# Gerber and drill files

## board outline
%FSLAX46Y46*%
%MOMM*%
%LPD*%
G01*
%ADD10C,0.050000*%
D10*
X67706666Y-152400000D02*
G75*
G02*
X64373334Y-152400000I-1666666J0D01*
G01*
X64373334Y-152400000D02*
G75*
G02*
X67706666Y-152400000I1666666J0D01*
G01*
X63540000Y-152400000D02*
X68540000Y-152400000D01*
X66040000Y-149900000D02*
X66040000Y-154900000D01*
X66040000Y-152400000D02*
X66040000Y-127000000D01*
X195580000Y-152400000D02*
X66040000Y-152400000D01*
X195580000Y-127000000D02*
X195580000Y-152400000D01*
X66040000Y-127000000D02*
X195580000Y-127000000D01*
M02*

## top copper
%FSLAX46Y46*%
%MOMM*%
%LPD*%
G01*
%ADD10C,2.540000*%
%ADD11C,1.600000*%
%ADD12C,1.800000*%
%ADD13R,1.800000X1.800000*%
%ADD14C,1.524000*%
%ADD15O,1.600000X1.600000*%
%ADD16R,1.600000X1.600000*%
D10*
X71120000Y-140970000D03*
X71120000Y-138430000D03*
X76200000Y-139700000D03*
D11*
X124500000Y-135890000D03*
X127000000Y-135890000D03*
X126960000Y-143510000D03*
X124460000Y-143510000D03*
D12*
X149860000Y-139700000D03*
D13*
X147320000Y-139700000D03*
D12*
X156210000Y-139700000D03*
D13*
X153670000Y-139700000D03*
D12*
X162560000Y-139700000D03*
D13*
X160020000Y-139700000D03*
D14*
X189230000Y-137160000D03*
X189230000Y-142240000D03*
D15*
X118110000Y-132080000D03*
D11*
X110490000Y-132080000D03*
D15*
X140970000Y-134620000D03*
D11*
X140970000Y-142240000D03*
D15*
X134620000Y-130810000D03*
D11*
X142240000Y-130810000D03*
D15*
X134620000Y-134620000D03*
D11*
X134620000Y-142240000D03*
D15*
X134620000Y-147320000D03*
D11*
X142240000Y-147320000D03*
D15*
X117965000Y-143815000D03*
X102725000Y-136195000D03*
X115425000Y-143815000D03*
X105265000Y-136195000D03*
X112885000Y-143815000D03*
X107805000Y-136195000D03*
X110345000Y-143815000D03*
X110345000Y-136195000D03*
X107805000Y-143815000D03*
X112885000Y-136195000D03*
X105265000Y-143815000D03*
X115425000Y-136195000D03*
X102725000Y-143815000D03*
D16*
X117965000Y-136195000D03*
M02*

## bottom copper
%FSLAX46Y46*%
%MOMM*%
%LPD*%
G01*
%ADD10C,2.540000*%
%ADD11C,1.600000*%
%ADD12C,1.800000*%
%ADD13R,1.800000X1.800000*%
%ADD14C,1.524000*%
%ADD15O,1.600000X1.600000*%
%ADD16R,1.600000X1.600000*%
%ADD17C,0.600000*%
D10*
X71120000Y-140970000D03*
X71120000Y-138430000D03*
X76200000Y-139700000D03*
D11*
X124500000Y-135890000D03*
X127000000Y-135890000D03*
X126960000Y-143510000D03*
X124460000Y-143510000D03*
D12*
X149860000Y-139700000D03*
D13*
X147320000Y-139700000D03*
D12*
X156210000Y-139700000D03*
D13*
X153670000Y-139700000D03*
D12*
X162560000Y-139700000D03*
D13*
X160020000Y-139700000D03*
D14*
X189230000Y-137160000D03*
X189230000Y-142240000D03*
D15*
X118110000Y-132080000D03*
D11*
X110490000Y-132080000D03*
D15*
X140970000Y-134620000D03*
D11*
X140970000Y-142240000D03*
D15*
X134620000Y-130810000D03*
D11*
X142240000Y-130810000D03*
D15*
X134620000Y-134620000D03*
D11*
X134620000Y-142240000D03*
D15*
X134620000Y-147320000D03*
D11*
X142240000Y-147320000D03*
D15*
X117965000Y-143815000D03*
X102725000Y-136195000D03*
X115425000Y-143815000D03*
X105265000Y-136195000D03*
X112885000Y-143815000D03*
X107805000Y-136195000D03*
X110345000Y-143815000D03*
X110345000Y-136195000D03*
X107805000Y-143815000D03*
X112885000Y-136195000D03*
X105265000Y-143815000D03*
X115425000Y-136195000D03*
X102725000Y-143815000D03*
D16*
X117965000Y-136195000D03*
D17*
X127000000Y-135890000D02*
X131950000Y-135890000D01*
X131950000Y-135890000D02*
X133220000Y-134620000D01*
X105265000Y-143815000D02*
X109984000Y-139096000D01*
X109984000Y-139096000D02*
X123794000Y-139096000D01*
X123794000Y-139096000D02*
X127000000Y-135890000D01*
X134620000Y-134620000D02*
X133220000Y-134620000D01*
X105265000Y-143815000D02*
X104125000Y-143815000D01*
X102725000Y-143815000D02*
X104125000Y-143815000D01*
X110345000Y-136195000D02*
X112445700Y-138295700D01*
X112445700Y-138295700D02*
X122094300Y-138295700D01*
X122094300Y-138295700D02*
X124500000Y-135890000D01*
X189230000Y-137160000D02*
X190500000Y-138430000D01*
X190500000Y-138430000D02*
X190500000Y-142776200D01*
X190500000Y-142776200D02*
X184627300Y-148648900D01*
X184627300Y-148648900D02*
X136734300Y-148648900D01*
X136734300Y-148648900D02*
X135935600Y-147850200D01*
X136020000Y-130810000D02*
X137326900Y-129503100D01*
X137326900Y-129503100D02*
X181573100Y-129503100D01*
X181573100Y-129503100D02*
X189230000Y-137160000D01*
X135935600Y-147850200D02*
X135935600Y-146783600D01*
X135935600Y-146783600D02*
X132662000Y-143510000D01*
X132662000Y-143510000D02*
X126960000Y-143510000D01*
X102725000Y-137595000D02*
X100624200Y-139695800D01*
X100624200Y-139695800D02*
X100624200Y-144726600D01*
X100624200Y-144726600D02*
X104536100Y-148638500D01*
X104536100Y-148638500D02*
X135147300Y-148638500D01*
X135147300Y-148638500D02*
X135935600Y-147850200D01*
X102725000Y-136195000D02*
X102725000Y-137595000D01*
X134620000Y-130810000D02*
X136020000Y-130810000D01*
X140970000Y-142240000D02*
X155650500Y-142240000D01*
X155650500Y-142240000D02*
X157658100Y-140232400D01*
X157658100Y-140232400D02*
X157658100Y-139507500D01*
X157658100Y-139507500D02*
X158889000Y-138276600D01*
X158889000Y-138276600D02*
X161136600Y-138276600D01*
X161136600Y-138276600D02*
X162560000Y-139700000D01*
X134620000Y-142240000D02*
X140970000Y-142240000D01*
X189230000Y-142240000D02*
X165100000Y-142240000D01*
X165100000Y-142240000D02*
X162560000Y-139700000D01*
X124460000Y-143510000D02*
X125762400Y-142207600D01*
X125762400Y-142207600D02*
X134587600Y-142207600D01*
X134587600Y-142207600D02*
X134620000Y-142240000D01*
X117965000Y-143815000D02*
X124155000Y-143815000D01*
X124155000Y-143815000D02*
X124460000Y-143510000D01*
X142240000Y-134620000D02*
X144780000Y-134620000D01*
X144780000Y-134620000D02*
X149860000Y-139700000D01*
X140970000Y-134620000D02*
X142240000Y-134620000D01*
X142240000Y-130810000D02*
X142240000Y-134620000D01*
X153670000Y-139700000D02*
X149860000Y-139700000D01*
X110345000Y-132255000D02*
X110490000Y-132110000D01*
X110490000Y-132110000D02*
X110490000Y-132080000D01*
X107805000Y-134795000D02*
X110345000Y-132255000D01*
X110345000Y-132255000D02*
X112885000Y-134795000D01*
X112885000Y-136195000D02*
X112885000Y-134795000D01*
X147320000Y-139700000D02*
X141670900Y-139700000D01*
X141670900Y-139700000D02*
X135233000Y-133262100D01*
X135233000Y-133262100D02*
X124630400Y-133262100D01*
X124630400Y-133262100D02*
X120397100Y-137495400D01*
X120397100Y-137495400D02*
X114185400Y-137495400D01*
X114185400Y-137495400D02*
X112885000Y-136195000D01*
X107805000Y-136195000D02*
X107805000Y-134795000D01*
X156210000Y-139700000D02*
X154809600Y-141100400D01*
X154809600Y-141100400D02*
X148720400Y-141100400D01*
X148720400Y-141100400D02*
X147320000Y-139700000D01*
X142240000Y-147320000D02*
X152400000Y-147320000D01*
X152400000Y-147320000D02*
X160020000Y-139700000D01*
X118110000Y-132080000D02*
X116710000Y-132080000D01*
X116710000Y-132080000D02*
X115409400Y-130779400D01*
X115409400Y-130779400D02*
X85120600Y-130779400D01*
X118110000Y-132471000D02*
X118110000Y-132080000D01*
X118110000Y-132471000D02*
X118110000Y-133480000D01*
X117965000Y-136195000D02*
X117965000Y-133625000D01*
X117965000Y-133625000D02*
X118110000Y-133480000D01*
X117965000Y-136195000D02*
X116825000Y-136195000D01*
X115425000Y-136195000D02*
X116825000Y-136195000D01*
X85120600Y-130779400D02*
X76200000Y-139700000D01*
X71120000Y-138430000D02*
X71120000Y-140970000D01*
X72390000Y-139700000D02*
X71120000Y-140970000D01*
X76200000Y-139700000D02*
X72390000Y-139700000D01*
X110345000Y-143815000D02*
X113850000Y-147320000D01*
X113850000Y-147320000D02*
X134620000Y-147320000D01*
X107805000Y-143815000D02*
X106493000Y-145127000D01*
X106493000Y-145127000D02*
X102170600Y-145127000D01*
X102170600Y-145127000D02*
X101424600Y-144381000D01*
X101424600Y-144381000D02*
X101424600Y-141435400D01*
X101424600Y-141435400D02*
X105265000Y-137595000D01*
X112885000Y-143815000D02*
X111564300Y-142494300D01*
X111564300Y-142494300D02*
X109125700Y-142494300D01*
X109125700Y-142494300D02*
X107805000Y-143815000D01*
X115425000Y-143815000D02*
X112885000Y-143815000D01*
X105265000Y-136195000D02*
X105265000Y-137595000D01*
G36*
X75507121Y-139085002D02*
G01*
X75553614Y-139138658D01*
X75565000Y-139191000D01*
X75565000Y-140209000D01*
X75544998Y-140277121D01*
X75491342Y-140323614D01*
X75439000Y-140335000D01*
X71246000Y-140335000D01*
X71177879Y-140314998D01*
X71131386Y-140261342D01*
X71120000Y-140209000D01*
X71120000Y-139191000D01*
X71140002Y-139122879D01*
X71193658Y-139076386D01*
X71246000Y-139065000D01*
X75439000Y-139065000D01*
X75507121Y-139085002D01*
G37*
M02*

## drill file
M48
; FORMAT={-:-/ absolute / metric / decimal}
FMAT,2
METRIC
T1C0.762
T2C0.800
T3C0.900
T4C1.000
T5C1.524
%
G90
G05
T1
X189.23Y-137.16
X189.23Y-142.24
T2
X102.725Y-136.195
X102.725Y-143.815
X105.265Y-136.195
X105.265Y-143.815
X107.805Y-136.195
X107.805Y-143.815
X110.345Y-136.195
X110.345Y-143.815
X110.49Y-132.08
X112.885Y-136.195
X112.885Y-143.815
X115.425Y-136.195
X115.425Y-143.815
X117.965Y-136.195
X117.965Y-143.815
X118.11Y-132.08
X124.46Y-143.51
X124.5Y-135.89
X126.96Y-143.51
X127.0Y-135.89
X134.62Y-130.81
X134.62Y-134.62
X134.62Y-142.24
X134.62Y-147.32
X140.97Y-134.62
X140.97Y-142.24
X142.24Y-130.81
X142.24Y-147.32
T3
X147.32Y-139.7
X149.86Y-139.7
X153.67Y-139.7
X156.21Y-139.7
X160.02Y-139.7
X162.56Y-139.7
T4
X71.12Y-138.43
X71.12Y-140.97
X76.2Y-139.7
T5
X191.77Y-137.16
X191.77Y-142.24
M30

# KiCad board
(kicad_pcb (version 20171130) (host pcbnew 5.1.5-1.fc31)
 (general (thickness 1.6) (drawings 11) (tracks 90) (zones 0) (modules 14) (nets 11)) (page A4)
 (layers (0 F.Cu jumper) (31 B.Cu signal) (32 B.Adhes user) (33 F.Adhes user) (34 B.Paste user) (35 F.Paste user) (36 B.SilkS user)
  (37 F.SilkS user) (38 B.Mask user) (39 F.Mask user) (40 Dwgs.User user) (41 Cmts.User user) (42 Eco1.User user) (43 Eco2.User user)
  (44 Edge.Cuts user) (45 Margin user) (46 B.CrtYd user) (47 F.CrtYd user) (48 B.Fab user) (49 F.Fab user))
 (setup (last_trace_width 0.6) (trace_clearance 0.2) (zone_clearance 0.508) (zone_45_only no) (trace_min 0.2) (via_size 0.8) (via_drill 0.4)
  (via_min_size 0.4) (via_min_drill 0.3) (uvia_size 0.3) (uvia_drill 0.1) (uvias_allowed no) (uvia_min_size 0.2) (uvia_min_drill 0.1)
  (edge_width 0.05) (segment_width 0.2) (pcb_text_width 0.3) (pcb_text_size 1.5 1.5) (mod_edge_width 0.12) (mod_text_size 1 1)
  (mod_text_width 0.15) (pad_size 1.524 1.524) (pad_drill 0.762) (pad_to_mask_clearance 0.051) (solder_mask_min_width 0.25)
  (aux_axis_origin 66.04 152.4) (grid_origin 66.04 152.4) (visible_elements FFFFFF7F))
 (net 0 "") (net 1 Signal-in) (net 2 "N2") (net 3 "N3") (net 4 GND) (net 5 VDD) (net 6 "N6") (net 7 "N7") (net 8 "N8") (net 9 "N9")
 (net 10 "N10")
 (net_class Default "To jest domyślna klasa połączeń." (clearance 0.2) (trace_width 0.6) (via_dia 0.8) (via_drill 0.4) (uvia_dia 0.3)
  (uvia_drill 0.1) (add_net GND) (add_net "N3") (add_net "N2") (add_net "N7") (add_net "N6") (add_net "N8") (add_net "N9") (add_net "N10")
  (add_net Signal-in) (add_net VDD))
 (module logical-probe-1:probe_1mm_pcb (layer F.Cu) (at 76.2 139.7)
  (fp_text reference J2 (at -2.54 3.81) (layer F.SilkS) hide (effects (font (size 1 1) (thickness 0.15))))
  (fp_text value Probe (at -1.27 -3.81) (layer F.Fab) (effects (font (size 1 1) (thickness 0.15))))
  (pad 1 thru_hole circle (at -5.08 1.27) (size 2.54 2.54) (drill 1) (layers B.Cu B.Mask) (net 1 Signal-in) (zone_connect 2))
  (pad 1 thru_hole circle (at -5.08 -1.27) (size 2.54 2.54) (drill 1) (layers B.Cu B.Mask) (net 1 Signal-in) (zone_connect 2))
  (pad 1 thru_hole circle (at 0 0) (size 2.54 2.54) (drill 1) (layers B.Cu B.Mask) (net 1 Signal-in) (zone_connect 2)))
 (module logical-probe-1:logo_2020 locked (layer F.Cu) (at 175.26 147.32)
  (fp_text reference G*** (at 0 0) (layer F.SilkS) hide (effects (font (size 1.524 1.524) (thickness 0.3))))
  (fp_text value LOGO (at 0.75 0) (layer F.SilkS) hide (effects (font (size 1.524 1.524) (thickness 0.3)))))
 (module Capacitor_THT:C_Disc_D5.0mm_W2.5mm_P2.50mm (layer F.Cu) (at 127 135.89 180)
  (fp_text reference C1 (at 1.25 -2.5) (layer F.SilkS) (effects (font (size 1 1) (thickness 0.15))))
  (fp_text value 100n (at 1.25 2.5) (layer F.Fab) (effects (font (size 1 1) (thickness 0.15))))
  (pad 2 thru_hole circle (at 2.5 0 180) (size 1.6 1.6) (drill 0.8) (layers *.Cu *.Mask) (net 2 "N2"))
  (pad 1 thru_hole circle (at 0 0 180) (size 1.6 1.6) (drill 0.8) (layers *.Cu *.Mask) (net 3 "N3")))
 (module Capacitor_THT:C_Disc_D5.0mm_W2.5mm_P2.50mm (layer F.Cu) (at 124.46 143.51)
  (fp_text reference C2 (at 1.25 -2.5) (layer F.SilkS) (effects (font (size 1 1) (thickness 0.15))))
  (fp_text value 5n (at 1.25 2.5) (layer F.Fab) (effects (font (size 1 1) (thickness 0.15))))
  (pad 2 thru_hole circle (at 2.5 0) (size 1.6 1.6) (drill 0.8) (layers *.Cu *.Mask) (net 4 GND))
  (pad 1 thru_hole circle (at 0 0) (size 1.6 1.6) (drill 0.8) (layers *.Cu *.Mask) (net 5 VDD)))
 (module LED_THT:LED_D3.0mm (layer F.Cu) (at 147.32 139.7)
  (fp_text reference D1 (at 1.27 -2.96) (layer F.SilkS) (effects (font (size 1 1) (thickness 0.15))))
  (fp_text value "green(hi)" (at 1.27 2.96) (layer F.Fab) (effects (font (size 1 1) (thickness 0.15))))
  (pad 2 thru_hole circle (at 2.54 0) (size 1.8 1.8) (drill 0.9) (layers *.Cu *.Mask) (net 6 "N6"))
  (pad 1 thru_hole rect (at 0 0) (size 1.8 1.8) (drill 0.9) (layers *.Cu *.Mask) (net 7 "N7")))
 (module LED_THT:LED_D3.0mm (layer F.Cu) (at 153.67 139.7)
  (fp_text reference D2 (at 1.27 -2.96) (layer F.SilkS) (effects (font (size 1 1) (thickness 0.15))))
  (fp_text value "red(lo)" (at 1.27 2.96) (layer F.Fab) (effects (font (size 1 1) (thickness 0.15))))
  (pad 2 thru_hole circle (at 2.54 0) (size 1.8 1.8) (drill 0.9) (layers *.Cu *.Mask) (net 7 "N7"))
  (pad 1 thru_hole rect (at 0 0) (size 1.8 1.8) (drill 0.9) (layers *.Cu *.Mask) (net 6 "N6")))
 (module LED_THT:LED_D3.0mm (layer F.Cu) (at 160.02 139.7)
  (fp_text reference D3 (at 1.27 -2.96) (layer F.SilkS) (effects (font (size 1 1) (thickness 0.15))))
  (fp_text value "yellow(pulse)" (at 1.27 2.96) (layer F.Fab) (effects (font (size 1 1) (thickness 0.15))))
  (pad 2 thru_hole circle (at 2.54 0) (size 1.8 1.8) (drill 0.9) (layers *.Cu *.Mask) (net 5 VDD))
  (pad 1 thru_hole rect (at 0 0) (size 1.8 1.8) (drill 0.9) (layers *.Cu *.Mask) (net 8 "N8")))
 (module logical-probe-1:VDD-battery (layer F.Cu) (at 189.23 139.7)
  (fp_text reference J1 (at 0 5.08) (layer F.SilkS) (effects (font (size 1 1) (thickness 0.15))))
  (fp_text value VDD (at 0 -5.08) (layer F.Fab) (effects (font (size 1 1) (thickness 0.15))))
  (pad "" np_thru_hole circle (at 2.54 2.54) (size 1.524 1.524) (drill 1.524) (layers *.Cu *.Mask))
  (pad "" np_thru_hole circle (at 2.54 -2.54) (size 1.524 1.524) (drill 1.524) (layers *.Cu *.Mask))
  (pad 2 thru_hole circle (at 0 -2.54) (size 1.524 1.524) (drill 0.762) (layers *.Cu *.Mask) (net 4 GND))
  (pad 1 thru_hole circle (at 0 2.54) (size 1.524 1.524) (drill 0.762) (layers *.Cu *.Mask) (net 5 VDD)))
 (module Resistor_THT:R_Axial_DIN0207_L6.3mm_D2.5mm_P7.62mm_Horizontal (layer F.Cu) (at 110.49 132.08)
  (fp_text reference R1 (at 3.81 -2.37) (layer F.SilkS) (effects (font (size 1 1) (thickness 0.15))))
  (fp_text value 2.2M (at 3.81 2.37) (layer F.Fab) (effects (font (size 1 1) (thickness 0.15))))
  (pad 2 thru_hole oval (at 7.62 0) (size 1.6 1.6) (drill 0.8) (layers *.Cu *.Mask) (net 1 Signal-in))
  (pad 1 thru_hole circle (at 0 0) (size 1.6 1.6) (drill 0.8) (layers *.Cu *.Mask) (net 7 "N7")))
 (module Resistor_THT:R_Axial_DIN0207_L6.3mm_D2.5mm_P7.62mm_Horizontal (layer F.Cu) (at 140.97 142.24 90)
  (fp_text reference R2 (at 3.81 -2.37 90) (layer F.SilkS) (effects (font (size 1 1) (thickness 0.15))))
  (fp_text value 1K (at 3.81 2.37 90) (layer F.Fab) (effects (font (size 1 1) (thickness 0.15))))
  (pad 2 thru_hole oval (at 7.62 0 90) (size 1.6 1.6) (drill 0.8) (layers *.Cu *.Mask) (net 6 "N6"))
  (pad 1 thru_hole circle (at 0 0 90) (size 1.6 1.6) (drill 0.8) (layers *.Cu *.Mask) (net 5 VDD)))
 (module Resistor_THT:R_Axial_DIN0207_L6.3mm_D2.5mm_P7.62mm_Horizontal (layer F.Cu) (at 142.24 130.81 180)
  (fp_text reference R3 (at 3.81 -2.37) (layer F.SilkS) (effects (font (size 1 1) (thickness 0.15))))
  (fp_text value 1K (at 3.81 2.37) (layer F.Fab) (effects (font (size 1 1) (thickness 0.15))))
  (pad 2 thru_hole oval (at 7.62 0 180) (size 1.6 1.6) (drill 0.8) (layers *.Cu *.Mask) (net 4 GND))
  (pad 1 thru_hole circle (at 0 0 180) (size 1.6 1.6) (drill 0.8) (layers *.Cu *.Mask) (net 6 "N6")))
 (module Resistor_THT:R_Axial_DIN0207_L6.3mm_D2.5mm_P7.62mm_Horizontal (layer F.Cu) (at 134.62 142.24 90)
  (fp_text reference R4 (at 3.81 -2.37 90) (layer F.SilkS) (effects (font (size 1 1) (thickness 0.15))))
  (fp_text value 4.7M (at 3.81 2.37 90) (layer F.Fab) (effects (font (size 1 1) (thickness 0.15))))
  (pad 2 thru_hole oval (at 7.62 0 90) (size 1.6 1.6) (drill 0.8) (layers *.Cu *.Mask) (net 3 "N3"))
  (pad 1 thru_hole circle (at 0 0 90) (size 1.6 1.6) (drill 0.8) (layers *.Cu *.Mask) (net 5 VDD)))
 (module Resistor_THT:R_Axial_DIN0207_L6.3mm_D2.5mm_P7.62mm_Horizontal (layer F.Cu) (at 142.24 147.32 180)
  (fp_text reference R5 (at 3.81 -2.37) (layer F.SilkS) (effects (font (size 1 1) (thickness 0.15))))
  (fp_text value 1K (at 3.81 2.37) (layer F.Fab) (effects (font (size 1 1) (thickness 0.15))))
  (pad 2 thru_hole oval (at 7.62 0 180) (size 1.6 1.6) (drill 0.8) (layers *.Cu *.Mask) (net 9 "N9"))
  (pad 1 thru_hole circle (at 0 0 180) (size 1.6 1.6) (drill 0.8) (layers *.Cu *.Mask) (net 8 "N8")))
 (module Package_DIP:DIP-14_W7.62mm (layer F.Cu) (at 117.965 136.195 270)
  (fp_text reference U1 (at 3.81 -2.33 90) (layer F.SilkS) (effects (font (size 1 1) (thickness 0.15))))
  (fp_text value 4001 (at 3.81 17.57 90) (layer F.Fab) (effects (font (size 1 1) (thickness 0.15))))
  (pad 14 thru_hole oval (at 7.62 0 270) (size 1.6 1.6) (drill 0.8) (layers *.Cu *.Mask) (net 5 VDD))
  (pad 7 thru_hole oval (at 0 15.24 270) (size 1.6 1.6) (drill 0.8) (layers *.Cu *.Mask) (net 4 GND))
  (pad 13 thru_hole oval (at 7.62 2.54 270) (size 1.6 1.6) (drill 0.8) (layers *.Cu *.Mask) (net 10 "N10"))
  (pad 6 thru_hole oval (at 0 12.7 270) (size 1.6 1.6) (drill 0.8) (layers *.Cu *.Mask) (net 10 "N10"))
  (pad 12 thru_hole oval (at 7.62 5.08 270) (size 1.6 1.6) (drill 0.8) (layers *.Cu *.Mask) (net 10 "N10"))
  (pad 5 thru_hole oval (at 0 10.16 270) (size 1.6 1.6) (drill 0.8) (layers *.Cu *.Mask) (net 7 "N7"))
  (pad 11 thru_hole oval (at 7.62 7.62 270) (size 1.6 1.6) (drill 0.8) (layers *.Cu *.Mask) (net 9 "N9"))
  (pad 4 thru_hole oval (at 0 7.62 270) (size 1.6 1.6) (drill 0.8) (layers *.Cu *.Mask) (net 2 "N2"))
  (pad 10 thru_hole oval (at 7.62 10.16 270) (size 1.6 1.6) (drill 0.8) (layers *.Cu *.Mask) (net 10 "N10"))
  (pad 3 thru_hole oval (at 0 5.08 270) (size 1.6 1.6) (drill 0.8) (layers *.Cu *.Mask) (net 7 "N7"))
  (pad 9 thru_hole oval (at 7.62 12.7 270) (size 1.6 1.6) (drill 0.8) (layers *.Cu *.Mask) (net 3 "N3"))
  (pad 2 thru_hole oval (at 0 2.54 270) (size 1.6 1.6) (drill 0.8) (layers *.Cu *.Mask) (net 1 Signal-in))
  (pad 8 thru_hole oval (at 7.62 15.24 270) (size 1.6 1.6) (drill 0.8) (layers *.Cu *.Mask) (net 3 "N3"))
  (pad 1 thru_hole rect (at 0 0 270) (size 1.6 1.6) (drill 0.8) (layers *.Cu *.Mask) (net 1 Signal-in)))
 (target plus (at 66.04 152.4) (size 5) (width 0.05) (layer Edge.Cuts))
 (gr_line (start 66.04 152.4) (end 66.04 127) (layer Edge.Cuts) (width 0.05))
 (gr_line (start 195.58 152.4) (end 66.04 152.4) (layer Edge.Cuts) (width 0.05))
 (gr_line (start 195.58 127) (end 195.58 152.4) (layer Edge.Cuts) (width 0.05))
 (gr_line (start 66.04 127) (end 195.58 127) (layer Edge.Cuts) (width 0.05))
 (segment (start 127 135.89) (end 131.95 135.89) (width 0.6) (layer B.Cu) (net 3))
 (segment (start 131.95 135.89) (end 133.22 134.62) (width 0.6) (layer B.Cu) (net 3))
 (segment (start 105.265 143.815) (end 109.984 139.096) (width 0.6) (layer B.Cu) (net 3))
 (segment (start 109.984 139.096) (end 123.794 139.096) (width 0.6) (layer B.Cu) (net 3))
 (segment (start 123.794 139.096) (end 127 135.89) (width 0.6) (layer B.Cu) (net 3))
 (segment (start 134.62 134.62) (end 133.22 134.62) (width 0.6) (layer B.Cu) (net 3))
 (segment (start 105.265 143.815) (end 104.125 143.815) (width 0.6) (layer B.Cu) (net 3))
 (segment (start 102.725 143.815) (end 104.125 143.815) (width 0.6) (layer B.Cu) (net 3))
 (segment (start 110.345 136.195) (end 112.4457 138.2957) (width 0.6) (layer B.Cu) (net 2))
 (segment (start 112.4457 138.2957) (end 122.0943 138.2957) (width 0.6) (layer B.Cu) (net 2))
 (segment (start 122.0943 138.2957) (end 124.5 135.89) (width 0.6) (layer B.Cu) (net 2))
 (segment (start 189.23 137.16) (end 190.5 138.43) (width 0.6) (layer B.Cu) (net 4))
 (segment (start 190.5 138.43) (end 190.5 142.7762) (width 0.6) (layer B.Cu) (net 4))
 (segment (start 190.5 142.7762) (end 184.6273 148.6489) (width 0.6) (layer B.Cu) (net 4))
 (segment (start 184.6273 148.6489) (end 136.7343 148.6489) (width 0.6) (layer B.Cu) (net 4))
 (segment (start 136.7343 148.6489) (end 135.9356 147.8502) (width 0.6) (layer B.Cu) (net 4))
 (segment (start 136.02 130.81) (end 137.3269 129.5031) (width 0.6) (layer B.Cu) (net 4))
 (segment (start 137.3269 129.5031) (end 181.5731 129.5031) (width 0.6) (layer B.Cu) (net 4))
 (segment (start 181.5731 129.5031) (end 189.23 137.16) (width 0.6) (layer B.Cu) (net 4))
 (segment (start 135.9356 147.8502) (end 135.9356 146.7836) (width 0.6) (layer B.Cu) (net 4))
 (segment (start 135.9356 146.7836) (end 132.662 143.51) (width 0.6) (layer B.Cu) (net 4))
 (segment (start 132.662 143.51) (end 126.96 143.51) (width 0.6) (layer B.Cu) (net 4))
 (segment (start 102.725 137.595) (end 100.6242 139.6958) (width 0.6) (layer B.Cu) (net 4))
 (segment (start 100.6242 139.6958) (end 100.6242 144.7266) (width 0.6) (layer B.Cu) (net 4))
 (segment (start 100.6242 144.7266) (end 104.5361 148.6385) (width 0.6) (layer B.Cu) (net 4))
 (segment (start 104.5361 148.6385) (end 135.1473 148.6385) (width 0.6) (layer B.Cu) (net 4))
 (segment (start 135.1473 148.6385) (end 135.9356 147.8502) (width 0.6) (layer B.Cu) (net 4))
 (segment (start 102.725 136.195) (end 102.725 137.595) (width 0.6) (layer B.Cu) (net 4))
 (segment (start 134.62 130.81) (end 136.02 130.81) (width 0.6) (layer B.Cu) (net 4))
 (segment (start 140.97 142.24) (end 155.6505 142.24) (width 0.6) (layer B.Cu) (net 5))
 (segment (start 155.6505 142.24) (end 157.6581 140.2324) (width 0.6) (layer B.Cu) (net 5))
 (segment (start 157.6581 140.2324) (end 157.6581 139.5075) (width 0.6) (layer B.Cu) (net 5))
 (segment (start 157.6581 139.5075) (end 158.889 138.2766) (width 0.6) (layer B.Cu) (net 5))
 (segment (start 158.889 138.2766) (end 161.1366 138.2766) (width 0.6) (layer B.Cu) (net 5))
 (segment (start 161.1366 138.2766) (end 162.56 139.7) (width 0.6) (layer B.Cu) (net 5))
 (segment (start 134.62 142.24) (end 140.97 142.24) (width 0.6) (layer B.Cu) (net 5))
 (segment (start 189.23 142.24) (end 165.1 142.24) (width 0.6) (layer B.Cu) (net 5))
 (segment (start 165.1 142.24) (end 162.56 139.7) (width 0.6) (layer B.Cu) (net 5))
 (segment (start 124.46 143.51) (end 125.7624 142.2076) (width 0.6) (layer B.Cu) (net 5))
 (segment (start 125.7624 142.2076) (end 134.5876 142.2076) (width 0.6) (layer B.Cu) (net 5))
 (segment (start 134.5876 142.2076) (end 134.62 142.24) (width 0.6) (layer B.Cu) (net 5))
 (segment (start 117.965 143.815) (end 124.155 143.815) (width 0.6) (layer B.Cu) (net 5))
 (segment (start 124.155 143.815) (end 124.46 143.51) (width 0.6) (layer B.Cu) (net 5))
 (segment (start 142.24 134.62) (end 144.78 134.62) (width 0.6) (layer B.Cu) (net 6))
 (segment (start 144.78 134.62) (end 149.86 139.7) (width 0.6) (layer B.Cu) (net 6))
 (segment (start 140.97 134.62) (end 142.24 134.62) (width 0.6) (layer B.Cu) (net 6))
 (segment (start 142.24 130.81) (end 142.24 134.62) (width 0.6) (layer B.Cu) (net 6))
 (segment (start 153.67 139.7) (end 149.86 139.7) (width 0.6) (layer B.Cu) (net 6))
 (segment (start 110.345 132.255) (end 110.49 132.11) (width 0.6) (layer B.Cu) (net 7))
 (segment (start 110.49 132.11) (end 110.49 132.08) (width 0.6) (layer B.Cu) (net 7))
 (segment (start 107.805 134.795) (end 110.345 132.255) (width 0.6) (layer B.Cu) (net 7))
 (segment (start 110.345 132.255) (end 112.885 134.795) (width 0.6) (layer B.Cu) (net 7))
 (segment (start 112.885 136.195) (end 112.885 134.795) (width 0.6) (layer B.Cu) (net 7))
 (segment (start 147.32 139.7) (end 141.6709 139.7) (width 0.6) (layer B.Cu) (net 7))
 (segment (start 141.6709 139.7) (end 135.233 133.2621) (width 0.6) (layer B.Cu) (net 7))
 (segment (start 135.233 133.2621) (end 124.6304 133.2621) (width 0.6) (layer B.Cu) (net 7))
 (segment (start 124.6304 133.2621) (end 120.3971 137.4954) (width 0.6) (layer B.Cu) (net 7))
 (segment (start 120.3971 137.4954) (end 114.1854 137.4954) (width 0.6) (layer B.Cu) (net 7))
 (segment (start 114.1854 137.4954) (end 112.885 136.195) (width 0.6) (layer B.Cu) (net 7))
 (segment (start 107.805 136.195) (end 107.805 134.795) (width 0.6) (layer B.Cu) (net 7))
 (segment (start 156.21 139.7) (end 154.8096 141.1004) (width 0.6) (layer B.Cu) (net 7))
 (segment (start 154.8096 141.1004) (end 148.7204 141.1004) (width 0.6) (layer B.Cu) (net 7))
 (segment (start 148.7204 141.1004) (end 147.32 139.7) (width 0.6) (layer B.Cu) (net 7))
 (segment (start 142.24 147.32) (end 152.4 147.32) (width 0.6) (layer B.Cu) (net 8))
 (segment (start 152.4 147.32) (end 160.02 139.7) (width 0.6) (layer B.Cu) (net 8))
 (segment (start 118.11 132.08) (end 116.71 132.08) (width 0.6) (layer B.Cu) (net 1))
 (segment (start 116.71 132.08) (end 115.4094 130.7794) (width 0.6) (layer B.Cu) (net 1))
 (segment (start 115.4094 130.7794) (end 85.1206 130.7794) (width 0.6) (layer B.Cu) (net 1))
 (segment (start 118.11 132.471) (end 118.11 132.08) (width 0.6) (layer B.Cu) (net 1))
 (segment (start 118.11 132.471) (end 118.11 133.48) (width 0.6) (layer B.Cu) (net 1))
 (segment (start 117.965 136.195) (end 117.965 133.625) (width 0.6) (layer B.Cu) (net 1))
 (segment (start 117.965 133.625) (end 118.11 133.48) (width 0.6) (layer B.Cu) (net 1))
 (segment (start 117.965 136.195) (end 116.825 136.195) (width 0.6) (layer B.Cu) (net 1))
 (segment (start 115.425 136.195) (end 116.825 136.195) (width 0.6) (layer B.Cu) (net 1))
 (segment (start 85.1206 130.7794) (end 76.2 139.7) (width 0.6) (layer B.Cu) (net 1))
 (segment (start 71.12 138.43) (end 71.12 140.97) (width 0.6) (layer B.Cu) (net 1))
 (segment (start 72.39 139.7) (end 71.12 140.97) (width 0.6) (layer B.Cu) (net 1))
 (segment (start 76.2 139.7) (end 72.39 139.7) (width 0.6) (layer B.Cu) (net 1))
 (segment (start 110.345 143.815) (end 113.85 147.32) (width 0.6) (layer B.Cu) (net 9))
 (segment (start 113.85 147.32) (end 134.62 147.32) (width 0.6) (layer B.Cu) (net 9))
 (segment (start 107.805 143.815) (end 106.493 145.127) (width 0.6) (layer B.Cu) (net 10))
 (segment (start 106.493 145.127) (end 102.1706 145.127) (width 0.6) (layer B.Cu) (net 10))
 (segment (start 102.1706 145.127) (end 101.4246 144.381) (width 0.6) (layer B.Cu) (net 10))
 (segment (start 101.4246 144.381) (end 101.4246 141.4354) (width 0.6) (layer B.Cu) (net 10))
 (segment (start 101.4246 141.4354) (end 105.265 137.595) (width 0.6) (layer B.Cu) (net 10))
 (segment (start 112.885 143.815) (end 111.5643 142.4943) (width 0.6) (layer B.Cu) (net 10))
 (segment (start 111.5643 142.4943) (end 109.1257 142.4943) (width 0.6) (layer B.Cu) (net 10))
 (segment (start 109.1257 142.4943) (end 107.805 143.815) (width 0.6) (layer B.Cu) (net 10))
 (segment (start 115.425 143.815) (end 112.885 143.815) (width 0.6) (layer B.Cu) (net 10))
 (segment (start 105.265 136.195) (end 105.265 137.595) (width 0.6) (layer B.Cu) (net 10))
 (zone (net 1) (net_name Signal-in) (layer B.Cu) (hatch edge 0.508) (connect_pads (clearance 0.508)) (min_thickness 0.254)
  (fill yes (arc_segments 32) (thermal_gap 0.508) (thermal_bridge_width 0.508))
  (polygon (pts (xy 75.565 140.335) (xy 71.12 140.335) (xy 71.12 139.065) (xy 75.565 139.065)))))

